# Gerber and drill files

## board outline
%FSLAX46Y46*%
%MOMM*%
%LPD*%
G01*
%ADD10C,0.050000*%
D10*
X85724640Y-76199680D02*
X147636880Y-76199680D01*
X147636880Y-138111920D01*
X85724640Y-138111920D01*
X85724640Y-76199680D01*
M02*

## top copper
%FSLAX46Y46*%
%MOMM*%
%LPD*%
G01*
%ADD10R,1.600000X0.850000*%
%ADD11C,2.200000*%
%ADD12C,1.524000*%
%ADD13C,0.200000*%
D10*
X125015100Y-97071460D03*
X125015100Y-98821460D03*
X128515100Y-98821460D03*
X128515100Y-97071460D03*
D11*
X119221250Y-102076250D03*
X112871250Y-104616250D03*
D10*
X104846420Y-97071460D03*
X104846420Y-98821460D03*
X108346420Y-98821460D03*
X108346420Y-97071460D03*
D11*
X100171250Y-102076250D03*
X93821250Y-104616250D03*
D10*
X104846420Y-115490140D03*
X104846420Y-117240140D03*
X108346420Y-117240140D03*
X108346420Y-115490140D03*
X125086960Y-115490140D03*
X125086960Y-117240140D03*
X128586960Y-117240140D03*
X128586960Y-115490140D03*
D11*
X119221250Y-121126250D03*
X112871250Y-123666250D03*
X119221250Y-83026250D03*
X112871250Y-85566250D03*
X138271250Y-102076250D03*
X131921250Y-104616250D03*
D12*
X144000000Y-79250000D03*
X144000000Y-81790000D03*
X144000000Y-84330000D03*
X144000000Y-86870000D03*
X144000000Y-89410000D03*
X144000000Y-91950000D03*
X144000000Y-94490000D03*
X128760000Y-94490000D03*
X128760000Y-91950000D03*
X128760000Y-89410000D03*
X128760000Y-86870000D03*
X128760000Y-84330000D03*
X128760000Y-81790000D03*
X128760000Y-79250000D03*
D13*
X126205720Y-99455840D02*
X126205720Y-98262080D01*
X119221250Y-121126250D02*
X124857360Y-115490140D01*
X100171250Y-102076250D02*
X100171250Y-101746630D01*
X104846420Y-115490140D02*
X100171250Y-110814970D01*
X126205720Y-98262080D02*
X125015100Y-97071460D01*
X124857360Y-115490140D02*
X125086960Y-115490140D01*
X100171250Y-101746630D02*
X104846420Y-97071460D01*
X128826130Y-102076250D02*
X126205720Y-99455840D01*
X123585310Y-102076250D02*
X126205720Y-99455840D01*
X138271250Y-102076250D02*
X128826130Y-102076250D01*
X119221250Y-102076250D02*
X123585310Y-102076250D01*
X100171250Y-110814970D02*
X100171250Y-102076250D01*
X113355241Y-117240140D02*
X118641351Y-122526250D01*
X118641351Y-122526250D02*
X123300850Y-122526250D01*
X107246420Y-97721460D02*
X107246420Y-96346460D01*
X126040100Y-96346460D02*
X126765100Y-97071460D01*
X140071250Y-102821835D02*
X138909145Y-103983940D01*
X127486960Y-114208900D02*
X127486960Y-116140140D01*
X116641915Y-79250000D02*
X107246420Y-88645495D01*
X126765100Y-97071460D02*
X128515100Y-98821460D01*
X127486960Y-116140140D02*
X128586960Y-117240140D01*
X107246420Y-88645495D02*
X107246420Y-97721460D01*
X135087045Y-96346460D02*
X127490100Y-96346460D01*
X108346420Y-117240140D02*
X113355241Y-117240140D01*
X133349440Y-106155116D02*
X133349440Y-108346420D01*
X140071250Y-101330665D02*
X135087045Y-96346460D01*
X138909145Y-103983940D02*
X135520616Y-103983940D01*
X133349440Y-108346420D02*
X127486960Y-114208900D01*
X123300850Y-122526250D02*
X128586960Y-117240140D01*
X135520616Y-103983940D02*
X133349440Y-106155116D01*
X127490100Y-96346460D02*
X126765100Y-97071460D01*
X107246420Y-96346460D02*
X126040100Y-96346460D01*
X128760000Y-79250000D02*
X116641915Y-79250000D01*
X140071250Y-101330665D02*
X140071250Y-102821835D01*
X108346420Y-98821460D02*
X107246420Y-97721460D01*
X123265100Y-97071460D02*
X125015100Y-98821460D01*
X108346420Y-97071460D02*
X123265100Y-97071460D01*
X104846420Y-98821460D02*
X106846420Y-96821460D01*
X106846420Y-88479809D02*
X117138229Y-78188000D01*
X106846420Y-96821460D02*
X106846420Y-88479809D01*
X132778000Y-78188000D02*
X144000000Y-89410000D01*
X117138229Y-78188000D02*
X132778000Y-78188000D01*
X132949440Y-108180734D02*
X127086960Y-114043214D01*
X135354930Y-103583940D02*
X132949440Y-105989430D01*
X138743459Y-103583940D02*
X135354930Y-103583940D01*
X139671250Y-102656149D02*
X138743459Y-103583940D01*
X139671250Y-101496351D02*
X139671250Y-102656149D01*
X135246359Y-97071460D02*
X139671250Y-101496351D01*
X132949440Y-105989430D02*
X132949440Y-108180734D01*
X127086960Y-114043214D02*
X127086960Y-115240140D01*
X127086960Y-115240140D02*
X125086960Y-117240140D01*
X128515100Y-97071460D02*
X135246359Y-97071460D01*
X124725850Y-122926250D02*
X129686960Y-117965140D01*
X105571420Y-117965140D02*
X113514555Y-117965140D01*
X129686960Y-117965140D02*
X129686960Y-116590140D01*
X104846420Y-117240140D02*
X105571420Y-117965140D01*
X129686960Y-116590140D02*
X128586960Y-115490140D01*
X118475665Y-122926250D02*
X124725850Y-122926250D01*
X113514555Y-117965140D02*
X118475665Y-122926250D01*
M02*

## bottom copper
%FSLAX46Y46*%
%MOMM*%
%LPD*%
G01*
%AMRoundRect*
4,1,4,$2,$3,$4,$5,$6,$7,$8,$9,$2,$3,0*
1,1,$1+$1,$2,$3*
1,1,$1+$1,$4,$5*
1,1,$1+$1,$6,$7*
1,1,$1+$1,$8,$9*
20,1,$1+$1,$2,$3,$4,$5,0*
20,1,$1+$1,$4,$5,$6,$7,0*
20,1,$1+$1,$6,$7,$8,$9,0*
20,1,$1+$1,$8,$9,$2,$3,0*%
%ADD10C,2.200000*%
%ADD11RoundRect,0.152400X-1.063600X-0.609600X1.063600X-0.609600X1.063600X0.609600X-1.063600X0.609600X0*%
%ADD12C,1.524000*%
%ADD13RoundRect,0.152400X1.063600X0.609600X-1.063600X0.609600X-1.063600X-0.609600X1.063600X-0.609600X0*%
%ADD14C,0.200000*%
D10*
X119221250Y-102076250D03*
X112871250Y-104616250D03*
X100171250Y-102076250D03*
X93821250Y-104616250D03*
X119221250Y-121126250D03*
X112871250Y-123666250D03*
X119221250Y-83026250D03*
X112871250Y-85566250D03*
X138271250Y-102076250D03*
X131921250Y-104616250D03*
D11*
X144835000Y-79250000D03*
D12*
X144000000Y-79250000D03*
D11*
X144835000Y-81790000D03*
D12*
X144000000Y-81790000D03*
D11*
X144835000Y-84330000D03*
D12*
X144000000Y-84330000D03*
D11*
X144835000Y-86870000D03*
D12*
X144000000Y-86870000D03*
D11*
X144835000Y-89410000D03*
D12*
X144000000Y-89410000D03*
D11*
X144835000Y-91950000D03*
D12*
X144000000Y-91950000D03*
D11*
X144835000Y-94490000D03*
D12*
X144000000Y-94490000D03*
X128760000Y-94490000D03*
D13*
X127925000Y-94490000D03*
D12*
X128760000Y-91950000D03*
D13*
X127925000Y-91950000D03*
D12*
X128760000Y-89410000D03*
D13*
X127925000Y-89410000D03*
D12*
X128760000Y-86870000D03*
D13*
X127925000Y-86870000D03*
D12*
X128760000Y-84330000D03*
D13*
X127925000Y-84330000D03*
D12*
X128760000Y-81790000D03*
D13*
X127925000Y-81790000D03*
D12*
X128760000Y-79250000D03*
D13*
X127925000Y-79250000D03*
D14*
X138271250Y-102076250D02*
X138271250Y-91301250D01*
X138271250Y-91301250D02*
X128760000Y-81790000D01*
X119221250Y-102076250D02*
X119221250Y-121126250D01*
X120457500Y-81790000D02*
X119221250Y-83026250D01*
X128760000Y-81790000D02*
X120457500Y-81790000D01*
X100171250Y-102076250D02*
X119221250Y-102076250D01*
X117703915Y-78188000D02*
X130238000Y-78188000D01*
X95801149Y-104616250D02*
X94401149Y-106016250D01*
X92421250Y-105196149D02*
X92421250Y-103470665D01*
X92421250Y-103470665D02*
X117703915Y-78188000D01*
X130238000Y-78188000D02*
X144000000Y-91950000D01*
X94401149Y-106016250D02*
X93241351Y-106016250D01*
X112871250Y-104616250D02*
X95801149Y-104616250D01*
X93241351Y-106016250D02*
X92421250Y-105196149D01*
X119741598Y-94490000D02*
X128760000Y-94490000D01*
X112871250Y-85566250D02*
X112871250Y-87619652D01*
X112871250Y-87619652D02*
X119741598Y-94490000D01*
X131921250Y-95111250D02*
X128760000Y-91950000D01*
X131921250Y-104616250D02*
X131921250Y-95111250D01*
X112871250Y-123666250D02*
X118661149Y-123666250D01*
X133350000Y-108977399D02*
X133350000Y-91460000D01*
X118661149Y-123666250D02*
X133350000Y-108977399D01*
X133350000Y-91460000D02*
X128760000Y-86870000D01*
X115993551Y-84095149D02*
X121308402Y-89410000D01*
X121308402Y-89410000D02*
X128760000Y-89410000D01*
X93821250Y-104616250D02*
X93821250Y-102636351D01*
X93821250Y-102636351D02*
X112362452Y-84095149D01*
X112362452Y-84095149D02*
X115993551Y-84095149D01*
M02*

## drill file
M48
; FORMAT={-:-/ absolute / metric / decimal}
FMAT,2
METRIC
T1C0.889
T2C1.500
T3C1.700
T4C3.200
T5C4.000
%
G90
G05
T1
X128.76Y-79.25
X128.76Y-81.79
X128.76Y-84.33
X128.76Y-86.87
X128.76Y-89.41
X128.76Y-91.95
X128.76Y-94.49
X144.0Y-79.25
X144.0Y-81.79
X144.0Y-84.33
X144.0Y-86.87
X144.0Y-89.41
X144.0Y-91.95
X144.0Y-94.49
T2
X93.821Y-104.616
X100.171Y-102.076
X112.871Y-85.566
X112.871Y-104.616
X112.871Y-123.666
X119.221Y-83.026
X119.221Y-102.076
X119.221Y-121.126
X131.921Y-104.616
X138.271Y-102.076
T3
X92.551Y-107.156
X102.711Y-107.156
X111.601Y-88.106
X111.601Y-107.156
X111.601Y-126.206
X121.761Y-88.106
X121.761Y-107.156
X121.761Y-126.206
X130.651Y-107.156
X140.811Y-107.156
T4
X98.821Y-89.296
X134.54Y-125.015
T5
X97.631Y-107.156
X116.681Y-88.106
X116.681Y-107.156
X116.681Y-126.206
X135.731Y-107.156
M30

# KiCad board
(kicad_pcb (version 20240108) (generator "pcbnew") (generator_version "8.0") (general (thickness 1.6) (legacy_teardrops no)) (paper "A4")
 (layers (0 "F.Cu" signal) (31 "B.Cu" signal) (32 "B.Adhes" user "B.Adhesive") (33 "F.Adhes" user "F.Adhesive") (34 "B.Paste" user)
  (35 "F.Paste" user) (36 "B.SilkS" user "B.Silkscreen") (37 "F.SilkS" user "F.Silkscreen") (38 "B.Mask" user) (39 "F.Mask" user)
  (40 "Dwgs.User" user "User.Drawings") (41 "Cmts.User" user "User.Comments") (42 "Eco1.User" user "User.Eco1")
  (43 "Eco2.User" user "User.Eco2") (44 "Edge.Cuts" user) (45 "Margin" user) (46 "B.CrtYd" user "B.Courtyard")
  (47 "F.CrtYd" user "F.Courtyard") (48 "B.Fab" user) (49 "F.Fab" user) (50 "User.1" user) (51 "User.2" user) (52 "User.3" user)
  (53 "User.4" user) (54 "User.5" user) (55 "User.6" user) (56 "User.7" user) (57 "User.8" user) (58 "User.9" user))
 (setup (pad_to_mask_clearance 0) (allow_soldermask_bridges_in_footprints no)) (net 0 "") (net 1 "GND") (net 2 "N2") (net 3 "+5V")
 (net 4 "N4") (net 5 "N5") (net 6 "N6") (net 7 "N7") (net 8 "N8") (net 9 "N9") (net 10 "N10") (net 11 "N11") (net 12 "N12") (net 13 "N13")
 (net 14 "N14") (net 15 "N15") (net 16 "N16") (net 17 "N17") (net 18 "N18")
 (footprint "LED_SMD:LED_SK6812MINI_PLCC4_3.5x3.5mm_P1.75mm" (layer "F.Cu") (at 126.7651 97.94646)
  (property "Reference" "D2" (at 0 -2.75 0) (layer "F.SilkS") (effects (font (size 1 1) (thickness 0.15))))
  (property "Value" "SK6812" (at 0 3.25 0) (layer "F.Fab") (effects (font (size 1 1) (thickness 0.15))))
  (pad "1" smd rect (at -1.75 -0.875) (size 1.6 0.85) (layers "F.Cu" "F.Paste" "F.Mask") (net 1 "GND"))
  (pad "2" smd rect (at -1.75 0.875) (size 1.6 0.85) (layers "F.Cu" "F.Paste" "F.Mask") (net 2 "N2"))
  (pad "3" smd rect (at 1.75 0.875) (size 1.6 0.85) (layers "F.Cu" "F.Paste" "F.Mask") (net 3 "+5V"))
  (pad "4" smd rect (at 1.75 -0.875) (size 1.6 0.85) (layers "F.Cu" "F.Paste" "F.Mask") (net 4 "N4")))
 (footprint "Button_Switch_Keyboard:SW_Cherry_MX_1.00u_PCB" (layer "F.Cu") (at 119.22125 102.07625)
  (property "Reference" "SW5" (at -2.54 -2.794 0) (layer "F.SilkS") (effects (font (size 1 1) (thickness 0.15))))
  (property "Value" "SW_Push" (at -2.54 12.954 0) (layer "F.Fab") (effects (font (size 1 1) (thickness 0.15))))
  (pad "" np_thru_hole circle (at -7.62 5.08) (size 1.7 1.7) (drill 1.7) (layers "*.Cu" "*.Mask"))
  (pad "" np_thru_hole circle (at -2.54 5.08) (size 4 4) (drill 4) (layers "*.Cu" "*.Mask"))
  (pad "" np_thru_hole circle (at 2.54 5.08) (size 1.7 1.7) (drill 1.7) (layers "*.Cu" "*.Mask"))
  (pad "1" thru_hole circle (at 0 0) (size 2.2 2.2) (drill 1.5) (layers "*.Cu" "*.Mask") (remove_unused_layers no) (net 1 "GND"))
  (pad "2" thru_hole circle (at -6.35 2.54) (size 2.2 2.2) (drill 1.5) (layers "*.Cu" "*.Mask") (remove_unused_layers no) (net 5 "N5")))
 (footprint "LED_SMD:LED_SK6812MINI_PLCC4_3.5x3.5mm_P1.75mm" (layer "F.Cu") (at 106.59642 97.94646)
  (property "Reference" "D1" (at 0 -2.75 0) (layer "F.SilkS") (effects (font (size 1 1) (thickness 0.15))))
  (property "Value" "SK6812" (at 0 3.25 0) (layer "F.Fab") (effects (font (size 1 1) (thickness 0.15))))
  (pad "1" smd rect (at -1.75 -0.875) (size 1.6 0.85) (layers "F.Cu" "F.Paste" "F.Mask") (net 1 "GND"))
  (pad "2" smd rect (at -1.75 0.875) (size 1.6 0.85) (layers "F.Cu" "F.Paste" "F.Mask") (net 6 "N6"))
  (pad "3" smd rect (at 1.75 0.875) (size 1.6 0.85) (layers "F.Cu" "F.Paste" "F.Mask") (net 3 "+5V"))
  (pad "4" smd rect (at 1.75 -0.875) (size 1.6 0.85) (layers "F.Cu" "F.Paste" "F.Mask") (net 2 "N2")))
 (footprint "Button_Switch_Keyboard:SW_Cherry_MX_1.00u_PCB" (layer "F.Cu") (at 100.17125 102.07625)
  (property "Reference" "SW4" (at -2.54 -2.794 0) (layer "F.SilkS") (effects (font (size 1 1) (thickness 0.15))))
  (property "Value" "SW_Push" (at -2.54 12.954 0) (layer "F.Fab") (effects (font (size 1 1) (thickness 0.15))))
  (pad "" np_thru_hole circle (at -7.62 5.08) (size 1.7 1.7) (drill 1.7) (layers "*.Cu" "*.Mask"))
  (pad "" np_thru_hole circle (at -2.54 5.08) (size 4 4) (drill 4) (layers "*.Cu" "*.Mask"))
  (pad "" np_thru_hole circle (at 2.54 5.08) (size 1.7 1.7) (drill 1.7) (layers "*.Cu" "*.Mask"))
  (pad "1" thru_hole circle (at 0 0) (size 2.2 2.2) (drill 1.5) (layers "*.Cu" "*.Mask") (remove_unused_layers no) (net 1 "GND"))
  (pad "2" thru_hole circle (at -6.35 2.54) (size 2.2 2.2) (drill 1.5) (layers "*.Cu" "*.Mask") (remove_unused_layers no) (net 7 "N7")))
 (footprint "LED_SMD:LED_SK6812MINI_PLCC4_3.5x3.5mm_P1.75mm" (layer "F.Cu") (at 106.59642 116.36514)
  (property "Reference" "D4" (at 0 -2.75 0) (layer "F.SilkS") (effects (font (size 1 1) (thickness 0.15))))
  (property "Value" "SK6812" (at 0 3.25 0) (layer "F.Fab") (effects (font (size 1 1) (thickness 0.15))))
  (pad "1" smd rect (at -1.75 -0.875) (size 1.6 0.85) (layers "F.Cu" "F.Paste" "F.Mask") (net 1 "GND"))
  (pad "2" smd rect (at -1.75 0.875) (size 1.6 0.85) (layers "F.Cu" "F.Paste" "F.Mask") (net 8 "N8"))
  (pad "3" smd rect (at 1.75 0.875) (size 1.6 0.85) (layers "F.Cu" "F.Paste" "F.Mask") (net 3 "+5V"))
  (pad "4" smd rect (at 1.75 -0.875) (size 1.6 0.85) (layers "F.Cu" "F.Paste" "F.Mask") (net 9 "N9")))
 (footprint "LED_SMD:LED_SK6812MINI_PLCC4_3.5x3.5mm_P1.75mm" (layer "F.Cu") (at 126.83696 116.36514)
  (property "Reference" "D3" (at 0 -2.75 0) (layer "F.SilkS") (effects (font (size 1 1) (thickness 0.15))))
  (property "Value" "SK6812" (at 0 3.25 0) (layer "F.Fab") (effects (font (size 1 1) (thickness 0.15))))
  (pad "1" smd rect (at -1.75 -0.875) (size 1.6 0.85) (layers "F.Cu" "F.Paste" "F.Mask") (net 1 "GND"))
  (pad "2" smd rect (at -1.75 0.875) (size 1.6 0.85) (layers "F.Cu" "F.Paste" "F.Mask") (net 4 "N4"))
  (pad "3" smd rect (at 1.75 0.875) (size 1.6 0.85) (layers "F.Cu" "F.Paste" "F.Mask") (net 3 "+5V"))
  (pad "4" smd rect (at 1.75 -0.875) (size 1.6 0.85) (layers "F.Cu" "F.Paste" "F.Mask") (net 8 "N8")))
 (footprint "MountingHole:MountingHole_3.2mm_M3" (layer "F.Cu") (at 98.82146 89.2965)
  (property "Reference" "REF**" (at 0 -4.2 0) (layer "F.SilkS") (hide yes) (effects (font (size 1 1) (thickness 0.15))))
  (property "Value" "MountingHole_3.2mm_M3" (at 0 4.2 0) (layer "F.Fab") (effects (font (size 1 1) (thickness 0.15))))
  (pad "" np_thru_hole circle (at 0 0) (size 3.2 3.2) (drill 3.2) (layers "*.Cu" "*.Mask")))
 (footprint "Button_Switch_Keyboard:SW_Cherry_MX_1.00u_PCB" (layer "F.Cu") (at 119.22125 121.12625)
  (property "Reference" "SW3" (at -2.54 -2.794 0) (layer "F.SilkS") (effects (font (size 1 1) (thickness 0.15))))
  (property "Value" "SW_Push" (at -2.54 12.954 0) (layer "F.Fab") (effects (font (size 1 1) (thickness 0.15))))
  (pad "" np_thru_hole circle (at -7.62 5.08) (size 1.7 1.7) (drill 1.7) (layers "*.Cu" "*.Mask"))
  (pad "" np_thru_hole circle (at -2.54 5.08) (size 4 4) (drill 4) (layers "*.Cu" "*.Mask"))
  (pad "" np_thru_hole circle (at 2.54 5.08) (size 1.7 1.7) (drill 1.7) (layers "*.Cu" "*.Mask"))
  (pad "1" thru_hole circle (at 0 0) (size 2.2 2.2) (drill 1.5) (layers "*.Cu" "*.Mask") (remove_unused_layers no) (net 1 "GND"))
  (pad "2" thru_hole circle (at -6.35 2.54) (size 2.2 2.2) (drill 1.5) (layers "*.Cu" "*.Mask") (remove_unused_layers no) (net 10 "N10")))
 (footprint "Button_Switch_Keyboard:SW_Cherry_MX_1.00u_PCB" (layer "F.Cu") (at 119.22125 83.02625)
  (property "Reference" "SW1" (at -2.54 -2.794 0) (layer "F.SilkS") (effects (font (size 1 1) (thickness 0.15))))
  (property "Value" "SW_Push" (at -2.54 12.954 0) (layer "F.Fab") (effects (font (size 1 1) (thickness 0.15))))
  (pad "" np_thru_hole circle (at -7.62 5.08) (size 1.7 1.7) (drill 1.7) (layers "*.Cu" "*.Mask"))
  (pad "" np_thru_hole circle (at -2.54 5.08) (size 4 4) (drill 4) (layers "*.Cu" "*.Mask"))
  (pad "" np_thru_hole circle (at 2.54 5.08) (size 1.7 1.7) (drill 1.7) (layers "*.Cu" "*.Mask"))
  (pad "1" thru_hole circle (at 0 0) (size 2.2 2.2) (drill 1.5) (layers "*.Cu" "*.Mask") (remove_unused_layers no) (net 1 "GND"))
  (pad "2" thru_hole circle (at -6.35 2.54) (size 2.2 2.2) (drill 1.5) (layers "*.Cu" "*.Mask") (remove_unused_layers no) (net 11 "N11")))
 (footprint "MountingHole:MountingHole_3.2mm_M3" (layer "F.Cu") (at 134.54006 125.0151)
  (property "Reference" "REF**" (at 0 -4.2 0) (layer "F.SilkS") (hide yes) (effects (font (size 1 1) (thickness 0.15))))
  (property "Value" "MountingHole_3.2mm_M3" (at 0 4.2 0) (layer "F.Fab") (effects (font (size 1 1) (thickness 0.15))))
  (pad "" np_thru_hole circle (at 0 0) (size 3.2 3.2) (drill 3.2) (layers "*.Cu" "*.Mask")))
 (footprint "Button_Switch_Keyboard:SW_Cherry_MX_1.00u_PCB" (layer "F.Cu") (at 138.27125 102.07625)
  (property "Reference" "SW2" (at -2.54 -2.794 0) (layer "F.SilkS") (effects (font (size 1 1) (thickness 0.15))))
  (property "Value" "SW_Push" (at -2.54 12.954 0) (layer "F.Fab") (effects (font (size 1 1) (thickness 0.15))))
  (pad "" np_thru_hole circle (at -7.62 5.08) (size 1.7 1.7) (drill 1.7) (layers "*.Cu" "*.Mask"))
  (pad "" np_thru_hole circle (at -2.54 5.08) (size 4 4) (drill 4) (layers "*.Cu" "*.Mask"))
  (pad "" np_thru_hole circle (at 2.54 5.08) (size 1.7 1.7) (drill 1.7) (layers "*.Cu" "*.Mask"))
  (pad "1" thru_hole circle (at 0 0) (size 2.2 2.2) (drill 1.5) (layers "*.Cu" "*.Mask") (remove_unused_layers no) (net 1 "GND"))
  (pad "2" thru_hole circle (at -6.35 2.54) (size 2.2 2.2) (drill 1.5) (layers "*.Cu" "*.Mask") (remove_unused_layers no) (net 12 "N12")))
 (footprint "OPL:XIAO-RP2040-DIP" (layer "B.Cu") (at 136.38 86.87 180)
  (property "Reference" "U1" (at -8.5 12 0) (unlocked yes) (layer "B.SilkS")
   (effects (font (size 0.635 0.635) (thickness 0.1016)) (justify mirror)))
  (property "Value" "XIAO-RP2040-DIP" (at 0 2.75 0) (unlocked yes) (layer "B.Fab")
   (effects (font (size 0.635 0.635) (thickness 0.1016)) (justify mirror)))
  (pad "1" smd roundrect (at -8.455 7.62) (size 2.432 1.524) (layers "B.Cu" "B.Mask") (roundrect_rratio 0.1) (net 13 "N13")
   (thermal_bridge_angle 45))
  (pad "1" thru_hole circle (at -7.62 7.62) (size 1.524 1.524) (drill 0.889) (layers "*.Cu" "*.Mask") (remove_unused_layers no)
   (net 13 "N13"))
  (pad "2" smd roundrect (at -8.455 5.08) (size 2.432 1.524) (layers "B.Cu" "B.Mask") (roundrect_rratio 0.1) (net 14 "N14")
   (thermal_bridge_angle 45))
  (pad "2" thru_hole circle (at -7.62 5.08) (size 1.524 1.524) (drill 0.889) (layers "*.Cu" "*.Mask") (remove_unused_layers no)
   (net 14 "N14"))
  (pad "3" smd roundrect (at -8.455 2.54) (size 2.432 1.524) (layers "B.Cu" "B.Mask") (roundrect_rratio 0.1) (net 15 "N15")
   (thermal_bridge_angle 45))
  (pad "3" thru_hole circle (at -7.62 2.54) (size 1.524 1.524) (drill 0.889) (layers "*.Cu" "*.Mask") (remove_unused_layers no)
   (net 15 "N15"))
  (pad "4" smd roundrect (at -8.455 0) (size 2.432 1.524) (layers "B.Cu" "B.Mask") (roundrect_rratio 0.1) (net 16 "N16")
   (thermal_bridge_angle 45))
  (pad "4" thru_hole circle (at -7.62 0) (size 1.524 1.524) (drill 0.889) (layers "*.Cu" "*.Mask") (remove_unused_layers no) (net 16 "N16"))
  (pad "5" smd roundrect (at -8.455 -2.54) (size 2.432 1.524) (layers "B.Cu" "B.Mask") (roundrect_rratio 0.1) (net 6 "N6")
   (thermal_bridge_angle 45))
  (pad "5" thru_hole circle (at -7.62 -2.54) (size 1.524 1.524) (drill 0.889) (layers "*.Cu" "*.Mask") (remove_unused_layers no)
   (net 6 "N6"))
  (pad "6" smd roundrect (at -8.455 -5.08) (size 2.432 1.524) (layers "B.Cu" "B.Mask") (roundrect_rratio 0.1) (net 5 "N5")
   (thermal_bridge_angle 45))
  (pad "6" thru_hole circle (at -7.62 -5.08) (size 1.524 1.524) (drill 0.889) (layers "*.Cu" "*.Mask") (remove_unused_layers no)
   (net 5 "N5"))
  (pad "7" smd roundrect (at -8.455 -7.62) (size 2.432 1.524) (layers "B.Cu" "B.Mask") (roundrect_rratio 0.1) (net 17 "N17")
   (thermal_bridge_angle 45))
  (pad "7" thru_hole circle (at -7.62 -7.62) (size 1.524 1.524) (drill 0.889) (layers "*.Cu" "*.Mask") (remove_unused_layers no)
   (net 17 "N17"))
  (pad "8" thru_hole circle (at 7.62 -7.62 180) (size 1.524 1.524) (drill 0.889) (layers "*.Cu" "*.Mask") (remove_unused_layers no)
   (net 11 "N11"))
  (pad "8" smd roundrect (at 8.455 -7.62 180) (size 2.432 1.524) (layers "B.Cu" "B.Mask") (roundrect_rratio 0.1) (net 11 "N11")
   (thermal_bridge_angle 45))
  (pad "9" thru_hole circle (at 7.62 -5.08 180) (size 1.524 1.524) (drill 0.889) (layers "*.Cu" "*.Mask") (remove_unused_layers no)
   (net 12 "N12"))
  (pad "9" smd roundrect (at 8.455 -5.08 180) (size 2.432 1.524) (layers "B.Cu" "B.Mask") (roundrect_rratio 0.1) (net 12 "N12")
   (thermal_bridge_angle 45))
  (pad "10" thru_hole circle (at 7.62 -2.54 180) (size 1.524 1.524) (drill 0.889) (layers "*.Cu" "*.Mask") (remove_unused_layers no)
   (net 7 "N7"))
  (pad "10" smd roundrect (at 8.455 -2.54 180) (size 2.432 1.524) (layers "B.Cu" "B.Mask") (roundrect_rratio 0.1) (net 7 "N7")
   (thermal_bridge_angle 45))
  (pad "11" thru_hole circle (at 7.62 0 180) (size 1.524 1.524) (drill 0.889) (layers "*.Cu" "*.Mask") (remove_unused_layers no)
   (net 10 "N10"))
  (pad "11" smd roundrect (at 8.455 0 180) (size 2.432 1.524) (layers "B.Cu" "B.Mask") (roundrect_rratio 0.1) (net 10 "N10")
   (thermal_bridge_angle 45))
  (pad "12" thru_hole circle (at 7.62 2.54 180) (size 1.524 1.524) (drill 0.889) (layers "*.Cu" "*.Mask") (remove_unused_layers no)
   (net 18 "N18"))
  (pad "12" smd roundrect (at 8.455 2.54 180) (size 2.432 1.524) (layers "B.Cu" "B.Mask") (roundrect_rratio 0.1) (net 18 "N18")
   (thermal_bridge_angle 45))
  (pad "13" thru_hole circle (at 7.62 5.08 180) (size 1.524 1.524) (drill 0.889) (layers "*.Cu" "*.Mask") (remove_unused_layers no)
   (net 1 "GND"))
  (pad "13" smd roundrect (at 8.455 5.08 180) (size 2.432 1.524) (layers "B.Cu" "B.Mask") (roundrect_rratio 0.1) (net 1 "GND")
   (thermal_bridge_angle 45))
  (pad "14" thru_hole circle (at 7.62 7.62 180) (size 1.524 1.524) (drill 0.889) (layers "*.Cu" "*.Mask") (remove_unused_layers no)
   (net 3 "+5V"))
  (pad "14" smd roundrect (at 8.455 7.62 180) (size 2.432 1.524) (layers "B.Cu" "B.Mask") (roundrect_rratio 0.1) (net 3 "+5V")
   (thermal_bridge_angle 45)))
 (gr_rect (start 85.72464 76.19968) (end 147.63688 138.11192) (stroke (width 0.05) (type default)) (fill none) (layer "Edge.Cuts"))
 (segment (start 126.20572 99.45584) (end 126.20572 98.26208) (width 0.2) (layer "F.Cu") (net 1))
 (segment (start 119.22125 121.12625) (end 124.85736 115.49014) (width 0.2) (layer "F.Cu") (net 1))
 (segment (start 100.17125 102.07625) (end 100.17125 101.74663) (width 0.2) (layer "F.Cu") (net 1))
 (segment (start 104.84642 115.49014) (end 100.17125 110.81497) (width 0.2) (layer "F.Cu") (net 1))
 (segment (start 126.20572 98.26208) (end 125.0151 97.07146) (width 0.2) (layer "F.Cu") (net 1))
 (segment (start 124.85736 115.49014) (end 125.08696 115.49014) (width 0.2) (layer "F.Cu") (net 1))
 (segment (start 100.17125 101.74663) (end 104.84642 97.07146) (width 0.2) (layer "F.Cu") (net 1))
 (segment (start 128.82613 102.07625) (end 126.20572 99.45584) (width 0.2) (layer "F.Cu") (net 1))
 (segment (start 123.58531 102.07625) (end 126.20572 99.45584) (width 0.2) (layer "F.Cu") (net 1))
 (segment (start 138.27125 102.07625) (end 128.82613 102.07625) (width 0.2) (layer "F.Cu") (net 1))
 (segment (start 119.22125 102.07625) (end 123.58531 102.07625) (width 0.2) (layer "F.Cu") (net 1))
 (segment (start 100.17125 110.81497) (end 100.17125 102.07625) (width 0.2) (layer "F.Cu") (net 1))
 (segment (start 138.27125 102.07625) (end 138.27125 91.30125) (width 0.2) (layer "B.Cu") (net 1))
 (segment (start 138.27125 91.30125) (end 128.76 81.79) (width 0.2) (layer "B.Cu") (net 1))
 (segment (start 119.22125 102.07625) (end 119.22125 121.12625) (width 0.2) (layer "B.Cu") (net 1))
 (segment (start 120.4575 81.79) (end 119.22125 83.02625) (width 0.2) (layer "B.Cu") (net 1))
 (segment (start 128.76 81.79) (end 120.4575 81.79) (width 0.2) (layer "B.Cu") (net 1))
 (segment (start 100.17125 102.07625) (end 119.22125 102.07625) (width 0.2) (layer "B.Cu") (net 1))
 (segment (start 113.355241 117.24014) (end 118.641351 122.52625) (width 0.2) (layer "F.Cu") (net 3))
 (segment (start 118.641351 122.52625) (end 123.30085 122.52625) (width 0.2) (layer "F.Cu") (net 3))
 (segment (start 107.24642 97.72146) (end 107.24642 96.34646) (width 0.2) (layer "F.Cu") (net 3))
 (segment (start 126.0401 96.34646) (end 126.7651 97.07146) (width 0.2) (layer "F.Cu") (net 3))
 (segment (start 140.07125 102.821835) (end 138.909145 103.98394) (width 0.2) (layer "F.Cu") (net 3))
 (segment (start 127.48696 114.2089) (end 127.48696 116.14014) (width 0.2) (layer "F.Cu") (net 3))
 (segment (start 116.641915 79.25) (end 107.24642 88.645495) (width 0.2) (layer "F.Cu") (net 3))
 (segment (start 126.7651 97.07146) (end 128.5151 98.82146) (width 0.2) (layer "F.Cu") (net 3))
 (segment (start 127.48696 116.14014) (end 128.58696 117.24014) (width 0.2) (layer "F.Cu") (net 3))
 (segment (start 107.24642 88.645495) (end 107.24642 97.72146) (width 0.2) (layer "F.Cu") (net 3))
 (segment (start 135.087045 96.34646) (end 127.4901 96.34646) (width 0.2) (layer "F.Cu") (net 3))
 (segment (start 108.34642 117.24014) (end 113.355241 117.24014) (width 0.2) (layer "F.Cu") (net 3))
 (segment (start 133.34944 106.155116) (end 133.34944 108.34642) (width 0.2) (layer "F.Cu") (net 3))
 (segment (start 140.07125 101.330665) (end 135.087045 96.34646) (width 0.2) (layer "F.Cu") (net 3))
 (segment (start 138.909145 103.98394) (end 135.520616 103.98394) (width 0.2) (layer "F.Cu") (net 3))
 (segment (start 133.34944 108.34642) (end 127.48696 114.2089) (width 0.2) (layer "F.Cu") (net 3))
 (segment (start 123.30085 122.52625) (end 128.58696 117.24014) (width 0.2) (layer "F.Cu") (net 3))
 (segment (start 135.520616 103.98394) (end 133.34944 106.155116) (width 0.2) (layer "F.Cu") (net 3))
 (segment (start 127.4901 96.34646) (end 126.7651 97.07146) (width 0.2) (layer "F.Cu") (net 3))
 (segment (start 107.24642 96.34646) (end 126.0401 96.34646) (width 0.2) (layer "F.Cu") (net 3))
 (segment (start 128.76 79.25) (end 116.641915 79.25) (width 0.2) (layer "F.Cu") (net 3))
 (segment (start 140.07125 101.330665) (end 140.07125 102.821835) (width 0.2) (layer "F.Cu") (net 3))
 (segment (start 108.34642 98.82146) (end 107.24642 97.72146) (width 0.2) (layer "F.Cu") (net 3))
 (segment (start 117.703915 78.188) (end 130.238 78.188) (width 0.2) (layer "B.Cu") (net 5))
 (segment (start 95.801149 104.61625) (end 94.401149 106.01625) (width 0.2) (layer "B.Cu") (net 5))
 (segment (start 92.42125 105.196149) (end 92.42125 103.470665) (width 0.2) (layer "B.Cu") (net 5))
 (segment (start 92.42125 103.470665) (end 117.703915 78.188) (width 0.2) (layer "B.Cu") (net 5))
 (segment (start 130.238 78.188) (end 144 91.95) (width 0.2) (layer "B.Cu") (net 5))
 (segment (start 94.401149 106.01625) (end 93.241351 106.01625) (width 0.2) (layer "B.Cu") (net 5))
 (segment (start 112.87125 104.61625) (end 95.801149 104.61625) (width 0.2) (layer "B.Cu") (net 5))
 (segment (start 93.241351 106.01625) (end 92.42125 105.196149) (width 0.2) (layer "B.Cu") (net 5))
 (segment (start 123.2651 97.07146) (end 125.0151 98.82146) (width 0.2) (layer "F.Cu") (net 2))
 (segment (start 108.34642 97.07146) (end 123.2651 97.07146) (width 0.2) (layer "F.Cu") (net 2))
 (segment (start 104.84642 98.82146) (end 106.84642 96.82146) (width 0.2) (layer "F.Cu") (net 6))
 (segment (start 106.84642 88.479809) (end 117.138229 78.188) (width 0.2) (layer "F.Cu") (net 6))
 (segment (start 106.84642 96.82146) (end 106.84642 88.479809) (width 0.2) (layer "F.Cu") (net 6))
 (segment (start 132.778 78.188) (end 144 89.41) (width 0.2) (layer "F.Cu") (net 6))
 (segment (start 117.138229 78.188) (end 132.778 78.188) (width 0.2) (layer "F.Cu") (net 6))
 (segment (start 119.741598 94.49) (end 128.76 94.49) (width 0.2) (layer "B.Cu") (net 11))
 (segment (start 112.87125 85.56625) (end 112.87125 87.619652) (width 0.2) (layer "B.Cu") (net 11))
 (segment (start 112.87125 87.619652) (end 119.741598 94.49) (width 0.2) (layer "B.Cu") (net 11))
 (segment (start 131.92125 95.11125) (end 128.76 91.95) (width 0.2) (layer "B.Cu") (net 12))
 (segment (start 131.92125 104.61625) (end 131.92125 95.11125) (width 0.2) (layer "B.Cu") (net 12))
 (segment (start 112.87125 123.66625) (end 118.661149 123.66625) (width 0.2) (layer "B.Cu") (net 10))
 (segment (start 133.35 108.977399) (end 133.35 91.46) (width 0.2) (layer "B.Cu") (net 10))
 (segment (start 118.661149 123.66625) (end 133.35 108.977399) (width 0.2) (layer "B.Cu") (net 10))
 (segment (start 133.35 91.46) (end 128.76 86.87) (width 0.2) (layer "B.Cu") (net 10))
 (segment (start 115.993551 84.095149) (end 121.308402 89.41) (width 0.2) (layer "B.Cu") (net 7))
 (segment (start 121.308402 89.41) (end 128.76 89.41) (width 0.2) (layer "B.Cu") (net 7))
 (segment (start 93.82125 104.61625) (end 93.82125 102.636351) (width 0.2) (layer "B.Cu") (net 7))
 (segment (start 93.82125 102.636351) (end 112.362452 84.095149) (width 0.2) (layer "B.Cu") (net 7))
 (segment (start 112.362452 84.095149) (end 115.993551 84.095149) (width 0.2) (layer "B.Cu") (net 7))
 (segment (start 132.94944 108.180734) (end 127.08696 114.043214) (width 0.2) (layer "F.Cu") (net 4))
 (segment (start 135.35493 103.58394) (end 132.94944 105.98943) (width 0.2) (layer "F.Cu") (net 4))
 (segment (start 138.743459 103.58394) (end 135.35493 103.58394) (width 0.2) (layer "F.Cu") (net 4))
 (segment (start 139.67125 102.656149) (end 138.743459 103.58394) (width 0.2) (layer "F.Cu") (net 4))
 (segment (start 139.67125 101.496351) (end 139.67125 102.656149) (width 0.2) (layer "F.Cu") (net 4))
 (segment (start 135.246359 97.07146) (end 139.67125 101.496351) (width 0.2) (layer "F.Cu") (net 4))
 (segment (start 132.94944 105.98943) (end 132.94944 108.180734) (width 0.2) (layer "F.Cu") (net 4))
 (segment (start 127.08696 114.043214) (end 127.08696 115.24014) (width 0.2) (layer "F.Cu") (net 4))
 (segment (start 127.08696 115.24014) (end 125.08696 117.24014) (width 0.2) (layer "F.Cu") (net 4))
 (segment (start 128.5151 97.07146) (end 135.246359 97.07146) (width 0.2) (layer "F.Cu") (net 4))
 (segment (start 124.72585 122.92625) (end 129.68696 117.96514) (width 0.2) (layer "F.Cu") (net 8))
 (segment (start 105.57142 117.96514) (end 113.514555 117.96514) (width 0.2) (layer "F.Cu") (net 8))
 (segment (start 129.68696 117.96514) (end 129.68696 116.59014) (width 0.2) (layer "F.Cu") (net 8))
 (segment (start 104.84642 117.24014) (end 105.57142 117.96514) (width 0.2) (layer "F.Cu") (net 8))
 (segment (start 129.68696 116.59014) (end 128.58696 115.49014) (width 0.2) (layer "F.Cu") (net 8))
 (segment (start 118.475665 122.92625) (end 124.72585 122.92625) (width 0.2) (layer "F.Cu") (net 8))
 (segment (start 113.514555 117.96514) (end 118.475665 122.92625) (width 0.2) (layer "F.Cu") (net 8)))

